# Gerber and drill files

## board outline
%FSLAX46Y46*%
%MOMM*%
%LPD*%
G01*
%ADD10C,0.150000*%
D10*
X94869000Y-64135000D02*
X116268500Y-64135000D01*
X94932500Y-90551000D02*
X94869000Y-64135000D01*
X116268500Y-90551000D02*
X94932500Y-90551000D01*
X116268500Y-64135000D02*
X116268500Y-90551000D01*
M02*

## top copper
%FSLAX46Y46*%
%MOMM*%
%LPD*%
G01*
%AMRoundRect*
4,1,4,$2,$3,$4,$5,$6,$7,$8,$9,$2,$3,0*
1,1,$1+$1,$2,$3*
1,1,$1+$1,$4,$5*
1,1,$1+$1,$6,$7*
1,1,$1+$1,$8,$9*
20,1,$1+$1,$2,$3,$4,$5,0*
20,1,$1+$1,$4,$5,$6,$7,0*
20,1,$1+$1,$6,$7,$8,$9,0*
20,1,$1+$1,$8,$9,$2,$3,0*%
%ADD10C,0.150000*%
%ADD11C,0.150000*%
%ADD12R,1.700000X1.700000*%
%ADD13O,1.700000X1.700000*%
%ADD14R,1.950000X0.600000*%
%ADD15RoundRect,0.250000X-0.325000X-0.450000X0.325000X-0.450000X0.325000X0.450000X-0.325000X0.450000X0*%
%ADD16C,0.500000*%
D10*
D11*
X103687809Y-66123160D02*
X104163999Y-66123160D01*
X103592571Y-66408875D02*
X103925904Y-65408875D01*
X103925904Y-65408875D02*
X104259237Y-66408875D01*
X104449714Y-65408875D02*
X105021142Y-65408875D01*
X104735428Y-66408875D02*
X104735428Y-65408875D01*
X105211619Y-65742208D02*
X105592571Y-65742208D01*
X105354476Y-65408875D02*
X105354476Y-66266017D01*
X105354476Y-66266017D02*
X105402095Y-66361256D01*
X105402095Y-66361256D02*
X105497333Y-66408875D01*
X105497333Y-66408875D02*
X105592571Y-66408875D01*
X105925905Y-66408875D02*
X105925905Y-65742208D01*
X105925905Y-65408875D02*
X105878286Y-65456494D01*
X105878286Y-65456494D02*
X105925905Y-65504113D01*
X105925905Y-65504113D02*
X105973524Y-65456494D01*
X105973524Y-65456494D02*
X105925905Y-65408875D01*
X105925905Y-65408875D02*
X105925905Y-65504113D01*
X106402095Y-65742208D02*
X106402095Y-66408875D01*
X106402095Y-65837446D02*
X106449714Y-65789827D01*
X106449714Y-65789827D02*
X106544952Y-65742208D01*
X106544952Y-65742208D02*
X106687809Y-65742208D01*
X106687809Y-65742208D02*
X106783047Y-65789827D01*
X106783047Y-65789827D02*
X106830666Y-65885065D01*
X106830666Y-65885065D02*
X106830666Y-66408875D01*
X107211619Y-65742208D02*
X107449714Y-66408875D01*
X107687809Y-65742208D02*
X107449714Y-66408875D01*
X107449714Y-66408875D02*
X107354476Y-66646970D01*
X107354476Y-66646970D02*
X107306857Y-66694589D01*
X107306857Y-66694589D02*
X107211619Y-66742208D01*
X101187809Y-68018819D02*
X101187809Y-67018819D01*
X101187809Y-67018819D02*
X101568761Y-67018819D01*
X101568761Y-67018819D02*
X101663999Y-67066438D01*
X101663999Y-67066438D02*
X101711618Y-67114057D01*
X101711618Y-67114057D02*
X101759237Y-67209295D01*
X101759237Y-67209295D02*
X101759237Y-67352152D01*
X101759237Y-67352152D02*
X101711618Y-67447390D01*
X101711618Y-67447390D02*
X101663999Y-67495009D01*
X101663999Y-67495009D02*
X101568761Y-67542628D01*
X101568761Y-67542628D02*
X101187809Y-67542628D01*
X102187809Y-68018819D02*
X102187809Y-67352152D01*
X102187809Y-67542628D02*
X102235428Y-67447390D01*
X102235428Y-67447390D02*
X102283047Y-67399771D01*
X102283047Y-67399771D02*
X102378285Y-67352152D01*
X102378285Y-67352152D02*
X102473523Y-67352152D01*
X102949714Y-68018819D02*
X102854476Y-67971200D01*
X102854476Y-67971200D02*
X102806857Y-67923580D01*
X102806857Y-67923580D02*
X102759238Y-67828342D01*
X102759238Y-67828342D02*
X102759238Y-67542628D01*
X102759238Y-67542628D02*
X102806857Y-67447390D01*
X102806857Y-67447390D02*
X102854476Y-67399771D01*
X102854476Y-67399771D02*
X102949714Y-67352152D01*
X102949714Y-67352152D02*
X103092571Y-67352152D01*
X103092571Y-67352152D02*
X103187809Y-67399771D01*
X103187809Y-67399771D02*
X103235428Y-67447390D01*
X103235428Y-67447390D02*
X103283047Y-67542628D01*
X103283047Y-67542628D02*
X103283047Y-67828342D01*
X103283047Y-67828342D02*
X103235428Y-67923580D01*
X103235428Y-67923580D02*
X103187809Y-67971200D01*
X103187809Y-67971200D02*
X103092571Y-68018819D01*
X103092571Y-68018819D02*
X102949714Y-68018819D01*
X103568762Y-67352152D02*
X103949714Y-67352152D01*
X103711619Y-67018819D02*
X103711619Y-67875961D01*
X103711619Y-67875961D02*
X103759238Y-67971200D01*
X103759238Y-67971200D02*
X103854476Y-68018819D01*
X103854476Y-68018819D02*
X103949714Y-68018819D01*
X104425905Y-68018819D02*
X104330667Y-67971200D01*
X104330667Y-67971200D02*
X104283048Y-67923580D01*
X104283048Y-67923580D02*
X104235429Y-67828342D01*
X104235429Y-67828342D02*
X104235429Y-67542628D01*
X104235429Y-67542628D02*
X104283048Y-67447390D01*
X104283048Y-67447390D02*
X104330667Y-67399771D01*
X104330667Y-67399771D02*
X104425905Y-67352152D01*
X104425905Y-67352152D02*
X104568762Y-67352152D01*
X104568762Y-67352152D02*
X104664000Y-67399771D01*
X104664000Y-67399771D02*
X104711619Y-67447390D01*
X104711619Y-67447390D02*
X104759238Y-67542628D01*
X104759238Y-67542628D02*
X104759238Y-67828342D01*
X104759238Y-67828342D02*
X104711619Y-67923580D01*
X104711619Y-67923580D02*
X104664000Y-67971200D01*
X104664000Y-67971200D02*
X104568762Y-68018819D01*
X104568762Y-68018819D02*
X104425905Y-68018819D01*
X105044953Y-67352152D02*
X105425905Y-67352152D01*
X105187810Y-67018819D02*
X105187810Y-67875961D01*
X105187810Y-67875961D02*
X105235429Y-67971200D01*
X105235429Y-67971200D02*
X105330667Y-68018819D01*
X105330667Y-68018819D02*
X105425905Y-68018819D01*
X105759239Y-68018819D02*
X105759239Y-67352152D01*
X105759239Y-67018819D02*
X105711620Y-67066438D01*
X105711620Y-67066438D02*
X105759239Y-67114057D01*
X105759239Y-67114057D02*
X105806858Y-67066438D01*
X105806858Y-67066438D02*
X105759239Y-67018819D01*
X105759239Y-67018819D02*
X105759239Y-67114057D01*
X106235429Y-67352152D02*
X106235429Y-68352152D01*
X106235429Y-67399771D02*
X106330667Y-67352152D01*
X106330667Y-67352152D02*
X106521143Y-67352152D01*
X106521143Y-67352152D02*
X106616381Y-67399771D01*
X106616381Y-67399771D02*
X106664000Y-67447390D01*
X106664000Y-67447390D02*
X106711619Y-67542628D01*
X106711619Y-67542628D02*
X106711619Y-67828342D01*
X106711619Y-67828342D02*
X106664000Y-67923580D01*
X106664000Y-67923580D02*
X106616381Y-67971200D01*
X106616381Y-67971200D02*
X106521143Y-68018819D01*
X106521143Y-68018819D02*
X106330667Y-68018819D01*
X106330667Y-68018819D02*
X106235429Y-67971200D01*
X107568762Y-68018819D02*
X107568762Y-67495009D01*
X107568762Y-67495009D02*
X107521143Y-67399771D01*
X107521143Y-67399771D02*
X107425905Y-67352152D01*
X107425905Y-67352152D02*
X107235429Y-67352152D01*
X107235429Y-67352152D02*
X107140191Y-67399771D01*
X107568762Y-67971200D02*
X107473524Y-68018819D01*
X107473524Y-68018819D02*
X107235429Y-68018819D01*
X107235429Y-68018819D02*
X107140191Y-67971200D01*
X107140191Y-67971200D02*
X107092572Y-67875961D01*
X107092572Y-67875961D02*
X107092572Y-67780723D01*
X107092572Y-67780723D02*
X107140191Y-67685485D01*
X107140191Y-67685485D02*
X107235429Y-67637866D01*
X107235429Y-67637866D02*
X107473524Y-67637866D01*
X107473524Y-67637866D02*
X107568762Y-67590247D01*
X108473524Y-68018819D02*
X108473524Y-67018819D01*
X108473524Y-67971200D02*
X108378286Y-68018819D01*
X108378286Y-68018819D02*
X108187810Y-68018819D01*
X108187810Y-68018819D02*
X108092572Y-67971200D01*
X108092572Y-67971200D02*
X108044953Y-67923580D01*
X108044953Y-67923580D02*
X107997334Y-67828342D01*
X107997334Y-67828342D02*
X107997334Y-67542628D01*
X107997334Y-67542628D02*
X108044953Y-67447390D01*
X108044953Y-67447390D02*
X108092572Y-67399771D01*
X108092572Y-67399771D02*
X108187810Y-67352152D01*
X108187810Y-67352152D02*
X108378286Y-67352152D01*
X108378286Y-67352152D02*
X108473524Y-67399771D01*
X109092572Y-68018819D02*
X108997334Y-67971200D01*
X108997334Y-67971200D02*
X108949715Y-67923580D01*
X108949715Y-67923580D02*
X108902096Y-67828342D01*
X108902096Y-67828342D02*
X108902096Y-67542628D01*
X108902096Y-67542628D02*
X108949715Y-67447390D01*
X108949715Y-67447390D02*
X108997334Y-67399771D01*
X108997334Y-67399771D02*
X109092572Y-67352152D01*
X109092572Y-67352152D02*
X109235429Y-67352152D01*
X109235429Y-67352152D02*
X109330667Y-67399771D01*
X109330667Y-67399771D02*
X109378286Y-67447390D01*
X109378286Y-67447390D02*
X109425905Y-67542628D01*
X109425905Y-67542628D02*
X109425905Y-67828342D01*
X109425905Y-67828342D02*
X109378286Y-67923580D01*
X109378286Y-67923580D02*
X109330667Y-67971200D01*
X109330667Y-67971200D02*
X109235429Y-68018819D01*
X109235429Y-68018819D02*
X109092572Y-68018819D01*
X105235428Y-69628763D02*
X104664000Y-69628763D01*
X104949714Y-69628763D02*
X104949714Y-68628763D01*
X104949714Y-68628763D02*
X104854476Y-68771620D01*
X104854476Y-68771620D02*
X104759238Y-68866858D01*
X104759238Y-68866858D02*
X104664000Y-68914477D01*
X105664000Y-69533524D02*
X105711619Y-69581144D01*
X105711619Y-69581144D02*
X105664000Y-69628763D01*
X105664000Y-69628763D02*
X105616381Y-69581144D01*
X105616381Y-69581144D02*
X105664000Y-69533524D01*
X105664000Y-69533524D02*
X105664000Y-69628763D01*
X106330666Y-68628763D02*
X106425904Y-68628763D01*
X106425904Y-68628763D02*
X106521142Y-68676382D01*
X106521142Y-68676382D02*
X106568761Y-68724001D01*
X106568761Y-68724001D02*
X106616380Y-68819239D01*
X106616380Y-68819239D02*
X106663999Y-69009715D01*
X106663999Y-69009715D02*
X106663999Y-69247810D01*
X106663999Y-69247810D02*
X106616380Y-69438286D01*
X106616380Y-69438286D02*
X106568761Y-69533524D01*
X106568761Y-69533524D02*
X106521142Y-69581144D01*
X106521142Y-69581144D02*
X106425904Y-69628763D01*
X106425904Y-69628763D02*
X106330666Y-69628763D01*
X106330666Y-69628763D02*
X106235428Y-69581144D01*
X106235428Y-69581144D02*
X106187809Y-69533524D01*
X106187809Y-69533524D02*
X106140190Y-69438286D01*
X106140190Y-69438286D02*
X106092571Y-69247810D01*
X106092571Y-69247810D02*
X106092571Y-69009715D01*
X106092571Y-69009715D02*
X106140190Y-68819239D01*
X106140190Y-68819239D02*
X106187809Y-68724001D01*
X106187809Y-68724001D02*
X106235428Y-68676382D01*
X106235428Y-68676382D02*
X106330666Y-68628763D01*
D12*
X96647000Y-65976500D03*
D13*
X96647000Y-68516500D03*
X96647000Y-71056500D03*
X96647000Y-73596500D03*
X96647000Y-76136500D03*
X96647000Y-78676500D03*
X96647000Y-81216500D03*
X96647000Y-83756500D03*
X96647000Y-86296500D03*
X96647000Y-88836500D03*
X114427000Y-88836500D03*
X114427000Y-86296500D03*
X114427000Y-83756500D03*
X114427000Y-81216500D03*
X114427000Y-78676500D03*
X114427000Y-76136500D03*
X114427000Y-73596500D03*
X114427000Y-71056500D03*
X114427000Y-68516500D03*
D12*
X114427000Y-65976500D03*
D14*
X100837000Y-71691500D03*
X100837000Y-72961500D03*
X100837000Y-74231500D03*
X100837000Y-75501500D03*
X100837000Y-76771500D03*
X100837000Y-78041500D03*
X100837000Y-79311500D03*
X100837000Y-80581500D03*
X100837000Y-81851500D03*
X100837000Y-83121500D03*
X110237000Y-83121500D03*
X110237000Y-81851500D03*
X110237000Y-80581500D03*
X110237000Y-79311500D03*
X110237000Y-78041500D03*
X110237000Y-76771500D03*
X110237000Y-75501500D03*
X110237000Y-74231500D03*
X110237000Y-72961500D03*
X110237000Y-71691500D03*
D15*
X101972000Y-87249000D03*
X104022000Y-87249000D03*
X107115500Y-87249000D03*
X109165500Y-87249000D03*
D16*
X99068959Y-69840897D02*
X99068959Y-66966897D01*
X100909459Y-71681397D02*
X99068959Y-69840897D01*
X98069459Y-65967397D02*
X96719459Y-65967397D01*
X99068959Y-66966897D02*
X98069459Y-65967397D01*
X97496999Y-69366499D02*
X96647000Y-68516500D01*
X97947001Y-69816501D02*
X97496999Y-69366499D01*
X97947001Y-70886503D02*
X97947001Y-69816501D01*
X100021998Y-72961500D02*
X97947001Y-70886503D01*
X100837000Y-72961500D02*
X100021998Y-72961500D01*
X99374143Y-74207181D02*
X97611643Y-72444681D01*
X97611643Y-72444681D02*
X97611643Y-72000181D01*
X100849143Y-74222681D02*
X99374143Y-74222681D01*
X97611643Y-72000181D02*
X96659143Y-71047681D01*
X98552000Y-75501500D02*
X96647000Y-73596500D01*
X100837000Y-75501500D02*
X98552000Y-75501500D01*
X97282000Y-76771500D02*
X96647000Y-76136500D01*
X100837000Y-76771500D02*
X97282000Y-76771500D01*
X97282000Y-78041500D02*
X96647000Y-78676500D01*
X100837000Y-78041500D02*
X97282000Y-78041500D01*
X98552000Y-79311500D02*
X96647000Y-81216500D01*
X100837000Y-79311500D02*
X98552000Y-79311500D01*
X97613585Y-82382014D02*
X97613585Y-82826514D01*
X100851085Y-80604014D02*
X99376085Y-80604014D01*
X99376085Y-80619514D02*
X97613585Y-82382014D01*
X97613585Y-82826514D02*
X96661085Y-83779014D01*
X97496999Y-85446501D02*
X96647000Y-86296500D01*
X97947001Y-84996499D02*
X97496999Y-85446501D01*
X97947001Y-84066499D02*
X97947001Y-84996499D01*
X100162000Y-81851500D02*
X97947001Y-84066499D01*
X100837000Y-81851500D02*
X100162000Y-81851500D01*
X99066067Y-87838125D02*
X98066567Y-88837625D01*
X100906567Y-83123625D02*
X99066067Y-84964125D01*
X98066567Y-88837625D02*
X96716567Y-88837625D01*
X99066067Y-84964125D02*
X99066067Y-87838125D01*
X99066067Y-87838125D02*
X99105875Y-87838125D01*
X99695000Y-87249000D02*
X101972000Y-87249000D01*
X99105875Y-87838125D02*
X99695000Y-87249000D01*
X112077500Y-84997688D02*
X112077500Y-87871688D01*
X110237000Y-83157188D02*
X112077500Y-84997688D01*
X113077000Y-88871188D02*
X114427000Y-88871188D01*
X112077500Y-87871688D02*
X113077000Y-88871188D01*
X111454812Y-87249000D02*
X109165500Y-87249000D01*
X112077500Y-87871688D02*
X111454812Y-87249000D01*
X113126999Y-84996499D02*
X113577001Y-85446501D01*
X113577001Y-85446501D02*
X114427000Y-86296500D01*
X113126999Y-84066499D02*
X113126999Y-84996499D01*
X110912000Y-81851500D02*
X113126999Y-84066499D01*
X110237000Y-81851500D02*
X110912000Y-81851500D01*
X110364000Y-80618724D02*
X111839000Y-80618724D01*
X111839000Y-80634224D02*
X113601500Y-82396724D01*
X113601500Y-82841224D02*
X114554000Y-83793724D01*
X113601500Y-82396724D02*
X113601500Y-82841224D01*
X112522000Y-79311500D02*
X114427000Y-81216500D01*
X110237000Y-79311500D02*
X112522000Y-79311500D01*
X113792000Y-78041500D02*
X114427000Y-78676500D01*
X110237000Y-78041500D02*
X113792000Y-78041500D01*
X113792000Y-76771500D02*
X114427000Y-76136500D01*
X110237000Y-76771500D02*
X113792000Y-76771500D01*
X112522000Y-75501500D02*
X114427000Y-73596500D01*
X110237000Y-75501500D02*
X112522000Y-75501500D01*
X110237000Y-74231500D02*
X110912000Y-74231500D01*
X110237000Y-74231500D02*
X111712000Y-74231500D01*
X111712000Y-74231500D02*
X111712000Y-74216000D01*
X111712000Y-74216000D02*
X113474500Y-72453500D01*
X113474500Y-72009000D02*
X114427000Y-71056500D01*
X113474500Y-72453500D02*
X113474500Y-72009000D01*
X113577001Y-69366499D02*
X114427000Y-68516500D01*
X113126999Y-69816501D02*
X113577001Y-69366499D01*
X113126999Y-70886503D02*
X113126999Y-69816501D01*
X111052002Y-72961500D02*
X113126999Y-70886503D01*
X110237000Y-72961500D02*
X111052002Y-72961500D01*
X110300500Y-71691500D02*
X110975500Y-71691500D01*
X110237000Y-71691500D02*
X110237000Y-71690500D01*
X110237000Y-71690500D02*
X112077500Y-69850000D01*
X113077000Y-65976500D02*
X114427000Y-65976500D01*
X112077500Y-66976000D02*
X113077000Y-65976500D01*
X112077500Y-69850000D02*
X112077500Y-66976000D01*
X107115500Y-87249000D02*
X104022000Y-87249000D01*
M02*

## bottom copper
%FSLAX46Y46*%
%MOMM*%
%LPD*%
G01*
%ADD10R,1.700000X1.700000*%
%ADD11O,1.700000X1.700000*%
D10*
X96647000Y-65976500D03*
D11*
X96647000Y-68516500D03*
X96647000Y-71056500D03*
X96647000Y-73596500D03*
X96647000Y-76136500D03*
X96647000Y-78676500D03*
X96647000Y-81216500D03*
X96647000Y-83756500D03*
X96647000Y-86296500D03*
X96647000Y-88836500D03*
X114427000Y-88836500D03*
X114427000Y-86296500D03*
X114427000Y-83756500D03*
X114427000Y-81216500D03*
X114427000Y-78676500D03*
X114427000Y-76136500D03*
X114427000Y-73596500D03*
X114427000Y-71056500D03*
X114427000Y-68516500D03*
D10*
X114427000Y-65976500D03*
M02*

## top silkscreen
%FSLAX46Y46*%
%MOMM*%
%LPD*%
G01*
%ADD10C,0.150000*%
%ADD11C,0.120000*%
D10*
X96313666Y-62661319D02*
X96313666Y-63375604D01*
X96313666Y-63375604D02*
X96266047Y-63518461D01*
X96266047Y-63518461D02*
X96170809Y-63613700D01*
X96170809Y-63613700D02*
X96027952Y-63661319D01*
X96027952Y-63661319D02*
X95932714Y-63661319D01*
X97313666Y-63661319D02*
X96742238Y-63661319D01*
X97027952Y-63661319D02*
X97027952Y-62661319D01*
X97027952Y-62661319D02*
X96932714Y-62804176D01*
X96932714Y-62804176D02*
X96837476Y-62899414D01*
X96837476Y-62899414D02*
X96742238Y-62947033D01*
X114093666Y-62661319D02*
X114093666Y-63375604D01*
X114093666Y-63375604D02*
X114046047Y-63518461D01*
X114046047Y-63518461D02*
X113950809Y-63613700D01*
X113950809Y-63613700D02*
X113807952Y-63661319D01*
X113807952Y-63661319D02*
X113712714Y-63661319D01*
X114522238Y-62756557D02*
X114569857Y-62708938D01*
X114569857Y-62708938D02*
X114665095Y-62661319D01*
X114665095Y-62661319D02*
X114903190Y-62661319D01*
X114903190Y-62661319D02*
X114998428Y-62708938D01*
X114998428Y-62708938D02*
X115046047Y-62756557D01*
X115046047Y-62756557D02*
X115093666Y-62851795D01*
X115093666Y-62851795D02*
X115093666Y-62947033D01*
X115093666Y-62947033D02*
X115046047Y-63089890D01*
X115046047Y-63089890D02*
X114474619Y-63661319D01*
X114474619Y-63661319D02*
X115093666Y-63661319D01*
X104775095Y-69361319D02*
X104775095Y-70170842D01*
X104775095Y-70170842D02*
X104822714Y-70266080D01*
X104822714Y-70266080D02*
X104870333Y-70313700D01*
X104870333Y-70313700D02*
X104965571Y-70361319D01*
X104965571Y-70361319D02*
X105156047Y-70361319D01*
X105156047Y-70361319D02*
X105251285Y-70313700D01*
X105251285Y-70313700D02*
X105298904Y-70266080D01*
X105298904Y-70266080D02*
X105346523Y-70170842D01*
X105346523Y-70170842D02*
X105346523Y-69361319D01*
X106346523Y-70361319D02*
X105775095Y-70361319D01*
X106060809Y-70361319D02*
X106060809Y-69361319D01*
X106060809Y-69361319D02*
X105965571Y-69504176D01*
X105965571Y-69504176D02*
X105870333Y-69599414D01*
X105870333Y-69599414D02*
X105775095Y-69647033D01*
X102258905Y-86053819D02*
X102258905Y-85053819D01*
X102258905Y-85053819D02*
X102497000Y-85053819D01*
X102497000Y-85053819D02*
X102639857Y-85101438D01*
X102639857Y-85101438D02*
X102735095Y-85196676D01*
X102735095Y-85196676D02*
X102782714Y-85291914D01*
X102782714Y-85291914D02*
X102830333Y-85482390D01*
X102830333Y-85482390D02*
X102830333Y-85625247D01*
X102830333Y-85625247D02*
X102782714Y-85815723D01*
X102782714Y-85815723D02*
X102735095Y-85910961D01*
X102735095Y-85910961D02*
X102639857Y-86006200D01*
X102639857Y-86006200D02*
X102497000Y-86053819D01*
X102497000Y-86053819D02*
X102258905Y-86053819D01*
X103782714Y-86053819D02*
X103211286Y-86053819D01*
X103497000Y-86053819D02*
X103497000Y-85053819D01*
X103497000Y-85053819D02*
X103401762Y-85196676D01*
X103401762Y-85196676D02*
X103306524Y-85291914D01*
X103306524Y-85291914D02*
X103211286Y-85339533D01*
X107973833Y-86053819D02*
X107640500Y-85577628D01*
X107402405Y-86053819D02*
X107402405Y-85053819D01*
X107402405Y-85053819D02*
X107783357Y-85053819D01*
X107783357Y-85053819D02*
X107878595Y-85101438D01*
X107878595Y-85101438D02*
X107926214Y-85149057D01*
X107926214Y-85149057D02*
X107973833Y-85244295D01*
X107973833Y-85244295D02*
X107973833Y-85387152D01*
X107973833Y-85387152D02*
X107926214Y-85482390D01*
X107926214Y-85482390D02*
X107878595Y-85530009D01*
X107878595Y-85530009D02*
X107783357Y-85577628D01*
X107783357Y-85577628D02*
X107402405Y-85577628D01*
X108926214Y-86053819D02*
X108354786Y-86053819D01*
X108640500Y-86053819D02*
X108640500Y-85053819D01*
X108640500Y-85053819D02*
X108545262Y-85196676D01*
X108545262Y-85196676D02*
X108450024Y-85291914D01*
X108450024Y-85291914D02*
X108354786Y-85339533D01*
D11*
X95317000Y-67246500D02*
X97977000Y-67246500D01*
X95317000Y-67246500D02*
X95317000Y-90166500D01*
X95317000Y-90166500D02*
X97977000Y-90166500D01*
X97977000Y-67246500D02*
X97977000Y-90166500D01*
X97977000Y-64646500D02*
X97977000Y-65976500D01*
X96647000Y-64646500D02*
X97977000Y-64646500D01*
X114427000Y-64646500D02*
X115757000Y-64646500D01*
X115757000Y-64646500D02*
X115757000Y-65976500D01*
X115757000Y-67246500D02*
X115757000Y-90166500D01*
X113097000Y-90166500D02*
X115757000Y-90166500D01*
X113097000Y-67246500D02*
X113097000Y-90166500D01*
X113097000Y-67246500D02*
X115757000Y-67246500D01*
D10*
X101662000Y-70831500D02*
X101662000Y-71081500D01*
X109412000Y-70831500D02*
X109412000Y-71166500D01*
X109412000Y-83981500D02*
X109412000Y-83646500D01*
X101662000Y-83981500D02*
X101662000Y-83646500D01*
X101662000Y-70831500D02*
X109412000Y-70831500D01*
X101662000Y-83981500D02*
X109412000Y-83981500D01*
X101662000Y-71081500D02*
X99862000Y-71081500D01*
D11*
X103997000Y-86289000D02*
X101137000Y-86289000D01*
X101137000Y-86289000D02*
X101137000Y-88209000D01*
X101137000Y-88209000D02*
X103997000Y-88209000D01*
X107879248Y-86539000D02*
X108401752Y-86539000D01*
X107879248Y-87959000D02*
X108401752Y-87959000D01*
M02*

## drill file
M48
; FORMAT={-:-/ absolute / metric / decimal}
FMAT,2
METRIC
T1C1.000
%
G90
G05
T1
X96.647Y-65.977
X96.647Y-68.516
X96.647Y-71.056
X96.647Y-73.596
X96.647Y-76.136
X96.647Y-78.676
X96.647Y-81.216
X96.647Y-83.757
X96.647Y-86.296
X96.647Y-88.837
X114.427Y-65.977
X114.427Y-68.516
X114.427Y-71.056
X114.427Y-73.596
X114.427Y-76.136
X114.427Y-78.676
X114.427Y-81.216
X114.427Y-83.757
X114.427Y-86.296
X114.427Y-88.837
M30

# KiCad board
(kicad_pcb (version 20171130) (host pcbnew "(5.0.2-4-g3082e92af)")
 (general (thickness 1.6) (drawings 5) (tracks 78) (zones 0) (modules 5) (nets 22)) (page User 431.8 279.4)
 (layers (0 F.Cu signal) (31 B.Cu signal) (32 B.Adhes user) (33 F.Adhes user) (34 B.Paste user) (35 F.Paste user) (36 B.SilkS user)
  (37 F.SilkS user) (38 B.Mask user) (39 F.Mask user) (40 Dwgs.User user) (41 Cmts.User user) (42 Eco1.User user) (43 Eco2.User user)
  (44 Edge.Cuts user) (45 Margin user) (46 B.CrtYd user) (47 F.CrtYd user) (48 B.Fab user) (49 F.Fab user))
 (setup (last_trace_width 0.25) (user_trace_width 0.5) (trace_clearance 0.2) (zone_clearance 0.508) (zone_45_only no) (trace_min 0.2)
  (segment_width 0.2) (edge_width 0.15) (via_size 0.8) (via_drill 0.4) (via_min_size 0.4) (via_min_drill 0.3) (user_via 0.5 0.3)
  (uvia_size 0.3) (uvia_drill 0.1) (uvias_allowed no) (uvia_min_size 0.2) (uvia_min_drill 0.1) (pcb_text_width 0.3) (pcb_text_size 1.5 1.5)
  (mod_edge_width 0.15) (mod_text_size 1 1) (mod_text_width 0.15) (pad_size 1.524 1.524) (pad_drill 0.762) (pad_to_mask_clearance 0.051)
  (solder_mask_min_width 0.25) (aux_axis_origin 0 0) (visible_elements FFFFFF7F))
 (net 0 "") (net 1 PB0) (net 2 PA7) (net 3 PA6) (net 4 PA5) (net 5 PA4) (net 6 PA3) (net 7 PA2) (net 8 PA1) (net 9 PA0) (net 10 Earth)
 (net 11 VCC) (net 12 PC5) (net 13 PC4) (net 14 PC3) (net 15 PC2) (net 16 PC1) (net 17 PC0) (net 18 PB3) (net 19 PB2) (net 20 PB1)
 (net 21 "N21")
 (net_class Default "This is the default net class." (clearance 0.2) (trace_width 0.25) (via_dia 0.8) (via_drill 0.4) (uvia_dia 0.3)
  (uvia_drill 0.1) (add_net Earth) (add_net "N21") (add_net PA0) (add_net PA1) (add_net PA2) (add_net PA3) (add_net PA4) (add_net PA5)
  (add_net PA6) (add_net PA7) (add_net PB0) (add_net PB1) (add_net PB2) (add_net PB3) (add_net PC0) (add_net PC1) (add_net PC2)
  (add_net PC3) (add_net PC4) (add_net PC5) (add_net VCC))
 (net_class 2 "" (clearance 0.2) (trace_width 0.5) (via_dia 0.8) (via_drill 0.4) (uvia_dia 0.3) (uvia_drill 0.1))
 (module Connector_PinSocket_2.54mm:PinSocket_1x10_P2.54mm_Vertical (layer F.Cu) (at 96.647 65.9765)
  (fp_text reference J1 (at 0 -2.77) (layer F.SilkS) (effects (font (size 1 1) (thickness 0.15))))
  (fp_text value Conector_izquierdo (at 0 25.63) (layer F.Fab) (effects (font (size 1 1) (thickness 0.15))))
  (fp_line (start -1.33 1.27) (end 1.33 1.27) (layer F.SilkS) (width 0.12))
  (fp_line (start -1.33 1.27) (end -1.33 24.19) (layer F.SilkS) (width 0.12))
  (fp_line (start -1.33 24.19) (end 1.33 24.19) (layer F.SilkS) (width 0.12))
  (fp_line (start 1.33 1.27) (end 1.33 24.19) (layer F.SilkS) (width 0.12))
  (fp_line (start 1.33 -1.33) (end 1.33 0) (layer F.SilkS) (width 0.12))
  (fp_line (start 0 -1.33) (end 1.33 -1.33) (layer F.SilkS) (width 0.12))
  (pad 1 thru_hole rect (at 0 0) (size 1.7 1.7) (drill 1) (layers *.Cu *.Mask) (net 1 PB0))
  (pad 2 thru_hole oval (at 0 2.54) (size 1.7 1.7) (drill 1) (layers *.Cu *.Mask) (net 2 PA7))
  (pad 3 thru_hole oval (at 0 5.08) (size 1.7 1.7) (drill 1) (layers *.Cu *.Mask) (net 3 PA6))
  (pad 4 thru_hole oval (at 0 7.62) (size 1.7 1.7) (drill 1) (layers *.Cu *.Mask) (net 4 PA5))
  (pad 5 thru_hole oval (at 0 10.16) (size 1.7 1.7) (drill 1) (layers *.Cu *.Mask) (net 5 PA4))
  (pad 6 thru_hole oval (at 0 12.7) (size 1.7 1.7) (drill 1) (layers *.Cu *.Mask) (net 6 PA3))
  (pad 7 thru_hole oval (at 0 15.24) (size 1.7 1.7) (drill 1) (layers *.Cu *.Mask) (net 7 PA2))
  (pad 8 thru_hole oval (at 0 17.78) (size 1.7 1.7) (drill 1) (layers *.Cu *.Mask) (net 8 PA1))
  (pad 9 thru_hole oval (at 0 20.32) (size 1.7 1.7) (drill 1) (layers *.Cu *.Mask) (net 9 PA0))
  (pad 10 thru_hole oval (at 0 22.86) (size 1.7 1.7) (drill 1) (layers *.Cu *.Mask) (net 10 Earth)))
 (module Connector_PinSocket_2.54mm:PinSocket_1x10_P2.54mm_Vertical (layer F.Cu) (at 114.427 65.9765)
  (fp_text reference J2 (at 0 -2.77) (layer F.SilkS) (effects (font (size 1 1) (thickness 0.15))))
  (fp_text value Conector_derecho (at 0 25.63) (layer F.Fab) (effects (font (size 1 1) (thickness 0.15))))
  (fp_line (start 0 -1.33) (end 1.33 -1.33) (layer F.SilkS) (width 0.12))
  (fp_line (start 1.33 -1.33) (end 1.33 0) (layer F.SilkS) (width 0.12))
  (fp_line (start 1.33 1.27) (end 1.33 24.19) (layer F.SilkS) (width 0.12))
  (fp_line (start -1.33 24.19) (end 1.33 24.19) (layer F.SilkS) (width 0.12))
  (fp_line (start -1.33 1.27) (end -1.33 24.19) (layer F.SilkS) (width 0.12))
  (fp_line (start -1.33 1.27) (end 1.33 1.27) (layer F.SilkS) (width 0.12))
  (pad 10 thru_hole oval (at 0 22.86) (size 1.7 1.7) (drill 1) (layers *.Cu *.Mask) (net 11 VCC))
  (pad 9 thru_hole oval (at 0 20.32) (size 1.7 1.7) (drill 1) (layers *.Cu *.Mask) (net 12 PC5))
  (pad 8 thru_hole oval (at 0 17.78) (size 1.7 1.7) (drill 1) (layers *.Cu *.Mask) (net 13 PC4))
  (pad 7 thru_hole oval (at 0 15.24) (size 1.7 1.7) (drill 1) (layers *.Cu *.Mask) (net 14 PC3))
  (pad 6 thru_hole oval (at 0 12.7) (size 1.7 1.7) (drill 1) (layers *.Cu *.Mask) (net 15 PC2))
  (pad 5 thru_hole oval (at 0 10.16) (size 1.7 1.7) (drill 1) (layers *.Cu *.Mask) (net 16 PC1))
  (pad 4 thru_hole oval (at 0 7.62) (size 1.7 1.7) (drill 1) (layers *.Cu *.Mask) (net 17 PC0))
  (pad 3 thru_hole oval (at 0 5.08) (size 1.7 1.7) (drill 1) (layers *.Cu *.Mask) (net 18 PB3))
  (pad 2 thru_hole oval (at 0 2.54) (size 1.7 1.7) (drill 1) (layers *.Cu *.Mask) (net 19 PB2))
  (pad 1 thru_hole rect (at 0 0) (size 1.7 1.7) (drill 1) (layers *.Cu *.Mask) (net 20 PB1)))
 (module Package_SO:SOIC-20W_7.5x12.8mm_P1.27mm (layer F.Cu) (at 105.537 77.4065)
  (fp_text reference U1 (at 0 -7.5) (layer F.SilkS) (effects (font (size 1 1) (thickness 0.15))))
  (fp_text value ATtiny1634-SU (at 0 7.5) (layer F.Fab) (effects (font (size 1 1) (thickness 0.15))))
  (fp_line (start -3.875 -6.575) (end -3.875 -6.325) (layer F.SilkS) (width 0.15))
  (fp_line (start 3.875 -6.575) (end 3.875 -6.24) (layer F.SilkS) (width 0.15))
  (fp_line (start 3.875 6.575) (end 3.875 6.24) (layer F.SilkS) (width 0.15))
  (fp_line (start -3.875 6.575) (end -3.875 6.24) (layer F.SilkS) (width 0.15))
  (fp_line (start -3.875 -6.575) (end 3.875 -6.575) (layer F.SilkS) (width 0.15))
  (fp_line (start -3.875 6.575) (end 3.875 6.575) (layer F.SilkS) (width 0.15))
  (fp_line (start -3.875 -6.325) (end -5.675 -6.325) (layer F.SilkS) (width 0.15))
  (pad 1 smd rect (at -4.7 -5.715) (size 1.95 0.6) (layers F.Cu F.Paste F.Mask) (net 1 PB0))
  (pad 2 smd rect (at -4.7 -4.445) (size 1.95 0.6) (layers F.Cu F.Paste F.Mask) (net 2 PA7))
  (pad 3 smd rect (at -4.7 -3.175) (size 1.95 0.6) (layers F.Cu F.Paste F.Mask) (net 3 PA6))
  (pad 4 smd rect (at -4.7 -1.905) (size 1.95 0.6) (layers F.Cu F.Paste F.Mask) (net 4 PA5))
  (pad 5 smd rect (at -4.7 -0.635) (size 1.95 0.6) (layers F.Cu F.Paste F.Mask) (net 5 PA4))
  (pad 6 smd rect (at -4.7 0.635) (size 1.95 0.6) (layers F.Cu F.Paste F.Mask) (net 6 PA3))
  (pad 7 smd rect (at -4.7 1.905) (size 1.95 0.6) (layers F.Cu F.Paste F.Mask) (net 7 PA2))
  (pad 8 smd rect (at -4.7 3.175) (size 1.95 0.6) (layers F.Cu F.Paste F.Mask) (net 8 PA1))
  (pad 9 smd rect (at -4.7 4.445) (size 1.95 0.6) (layers F.Cu F.Paste F.Mask) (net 9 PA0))
  (pad 10 smd rect (at -4.7 5.715) (size 1.95 0.6) (layers F.Cu F.Paste F.Mask) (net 10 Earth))
  (pad 11 smd rect (at 4.7 5.715) (size 1.95 0.6) (layers F.Cu F.Paste F.Mask) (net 11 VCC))
  (pad 12 smd rect (at 4.7 4.445) (size 1.95 0.6) (layers F.Cu F.Paste F.Mask) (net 12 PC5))
  (pad 13 smd rect (at 4.7 3.175) (size 1.95 0.6) (layers F.Cu F.Paste F.Mask) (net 13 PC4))
  (pad 14 smd rect (at 4.7 1.905) (size 1.95 0.6) (layers F.Cu F.Paste F.Mask) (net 14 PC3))
  (pad 15 smd rect (at 4.7 0.635) (size 1.95 0.6) (layers F.Cu F.Paste F.Mask) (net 15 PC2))
  (pad 16 smd rect (at 4.7 -0.635) (size 1.95 0.6) (layers F.Cu F.Paste F.Mask) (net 16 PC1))
  (pad 17 smd rect (at 4.7 -1.905) (size 1.95 0.6) (layers F.Cu F.Paste F.Mask) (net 17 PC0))
  (pad 18 smd rect (at 4.7 -3.175) (size 1.95 0.6) (layers F.Cu F.Paste F.Mask) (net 18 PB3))
  (pad 19 smd rect (at 4.7 -4.445) (size 1.95 0.6) (layers F.Cu F.Paste F.Mask) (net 19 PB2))
  (pad 20 smd rect (at 4.7 -5.715) (size 1.95 0.6) (layers F.Cu F.Paste F.Mask) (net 20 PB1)))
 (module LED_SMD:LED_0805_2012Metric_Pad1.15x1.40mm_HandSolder (layer F.Cu) (at 102.997 87.249)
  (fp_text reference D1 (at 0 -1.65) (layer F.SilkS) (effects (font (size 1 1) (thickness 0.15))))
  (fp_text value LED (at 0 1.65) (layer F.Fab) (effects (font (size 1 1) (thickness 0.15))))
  (fp_line (start 1 -0.96) (end -1.86 -0.96) (layer F.SilkS) (width 0.12))
  (fp_line (start -1.86 -0.96) (end -1.86 0.96) (layer F.SilkS) (width 0.12))
  (fp_line (start -1.86 0.96) (end 1 0.96) (layer F.SilkS) (width 0.12))
  (pad 1 smd roundrect (at -1.025 0) (size 1.15 1.4) (layers F.Cu F.Paste F.Mask) (roundrect_rratio 0.217391) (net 10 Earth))
  (pad 2 smd roundrect (at 1.025 0) (size 1.15 1.4) (layers F.Cu F.Paste F.Mask) (roundrect_rratio 0.217391) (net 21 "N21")))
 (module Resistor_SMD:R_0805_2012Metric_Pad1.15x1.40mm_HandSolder (layer F.Cu) (at 108.1405 87.249)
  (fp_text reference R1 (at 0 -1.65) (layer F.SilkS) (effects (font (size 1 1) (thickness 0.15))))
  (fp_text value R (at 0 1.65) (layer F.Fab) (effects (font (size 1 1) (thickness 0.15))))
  (fp_line (start -0.261252 -0.71) (end 0.261252 -0.71) (layer F.SilkS) (width 0.12))
  (fp_line (start -0.261252 0.71) (end 0.261252 0.71) (layer F.SilkS) (width 0.12))
  (pad 1 smd roundrect (at -1.025 0) (size 1.15 1.4) (layers F.Cu F.Paste F.Mask) (roundrect_rratio 0.217391) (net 21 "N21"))
  (pad 2 smd roundrect (at 1.025 0) (size 1.15 1.4) (layers F.Cu F.Paste F.Mask) (roundrect_rratio 0.217391) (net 11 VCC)))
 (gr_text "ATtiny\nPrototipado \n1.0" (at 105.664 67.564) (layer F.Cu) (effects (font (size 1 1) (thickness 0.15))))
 (gr_line (start 94.869 64.135) (end 116.2685 64.135) (layer Edge.Cuts) (width 0.15))
 (gr_line (start 94.9325 90.551) (end 94.869 64.135) (layer Edge.Cuts) (width 0.15))
 (gr_line (start 116.2685 90.551) (end 94.9325 90.551) (layer Edge.Cuts) (width 0.15))
 (gr_line (start 116.2685 64.135) (end 116.2685 90.551) (layer Edge.Cuts) (width 0.15))
 (segment (start 99.068959 69.840897) (end 99.068959 66.966897) (width 0.5) (layer F.Cu) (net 1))
 (segment (start 100.909459 71.681397) (end 99.068959 69.840897) (width 0.5) (layer F.Cu) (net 1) (status 10))
 (segment (start 98.069459 65.967397) (end 96.719459 65.967397) (width 0.5) (layer F.Cu) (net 1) (status 20))
 (segment (start 99.068959 66.966897) (end 98.069459 65.967397) (width 0.5) (layer F.Cu) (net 1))
 (segment (start 97.496999 69.366499) (end 96.647 68.5165) (width 0.5) (layer F.Cu) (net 2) (status 30))
 (segment (start 97.947001 69.816501) (end 97.496999 69.366499) (width 0.5) (layer F.Cu) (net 2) (status 20))
 (segment (start 97.947001 70.886503) (end 97.947001 69.816501) (width 0.5) (layer F.Cu) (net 2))
 (segment (start 100.021998 72.9615) (end 97.947001 70.886503) (width 0.5) (layer F.Cu) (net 2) (status 10))
 (segment (start 100.837 72.9615) (end 100.021998 72.9615) (width 0.5) (layer F.Cu) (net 2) (status 30))
 (segment (start 99.374143 74.207181) (end 97.611643 72.444681) (width 0.5) (layer F.Cu) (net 3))
 (segment (start 97.611643 72.444681) (end 97.611643 72.000181) (width 0.5) (layer F.Cu) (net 3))
 (segment (start 100.849143 74.222681) (end 99.374143 74.222681) (width 0.5) (layer F.Cu) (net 3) (status 10))
 (segment (start 97.611643 72.000181) (end 96.659143 71.047681) (width 0.5) (layer F.Cu) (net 3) (status 20))
 (segment (start 98.552 75.5015) (end 96.647 73.5965) (width 0.5) (layer F.Cu) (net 4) (status 20))
 (segment (start 100.837 75.5015) (end 98.552 75.5015) (width 0.5) (layer F.Cu) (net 4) (status 10))
 (segment (start 97.282 76.7715) (end 96.647 76.1365) (width 0.5) (layer F.Cu) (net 5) (status 30))
 (segment (start 100.837 76.7715) (end 97.282 76.7715) (width 0.5) (layer F.Cu) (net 5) (status 30))
 (segment (start 97.282 78.0415) (end 96.647 78.6765) (width 0.5) (layer F.Cu) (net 6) (status 30))
 (segment (start 100.837 78.0415) (end 97.282 78.0415) (width 0.5) (layer F.Cu) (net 6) (status 30))
 (segment (start 98.552 79.3115) (end 96.647 81.2165) (width 0.5) (layer F.Cu) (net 7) (status 20))
 (segment (start 100.837 79.3115) (end 98.552 79.3115) (width 0.5) (layer F.Cu) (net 7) (status 10))
 (segment (start 97.613585 82.382014) (end 97.613585 82.826514) (width 0.5) (layer F.Cu) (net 8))
 (segment (start 100.851085 80.604014) (end 99.376085 80.604014) (width 0.5) (layer F.Cu) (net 8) (status 10))
 (segment (start 99.376085 80.619514) (end 97.613585 82.382014) (width 0.5) (layer F.Cu) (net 8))
 (segment (start 97.613585 82.826514) (end 96.661085 83.779014) (width 0.5) (layer F.Cu) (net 8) (status 20))
 (segment (start 97.496999 85.446501) (end 96.647 86.2965) (width 0.5) (layer F.Cu) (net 9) (status 30))
 (segment (start 97.947001 84.996499) (end 97.496999 85.446501) (width 0.5) (layer F.Cu) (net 9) (status 20))
 (segment (start 97.947001 84.066499) (end 97.947001 84.996499) (width 0.5) (layer F.Cu) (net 9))
 (segment (start 100.162 81.8515) (end 97.947001 84.066499) (width 0.5) (layer F.Cu) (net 9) (status 10))
 (segment (start 100.837 81.8515) (end 100.162 81.8515) (width 0.5) (layer F.Cu) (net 9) (status 30))
 (segment (start 99.066067 87.838125) (end 98.066567 88.837625) (width 0.5) (layer F.Cu) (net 10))
 (segment (start 100.906567 83.123625) (end 99.066067 84.964125) (width 0.5) (layer F.Cu) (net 10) (status 10))
 (segment (start 98.066567 88.837625) (end 96.716567 88.837625) (width 0.5) (layer F.Cu) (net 10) (status 20))
 (segment (start 99.066067 84.964125) (end 99.066067 87.838125) (width 0.5) (layer F.Cu) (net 10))
 (segment (start 99.066067 87.838125) (end 99.105875 87.838125) (width 0.5) (layer F.Cu) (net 10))
 (segment (start 99.695 87.249) (end 101.972 87.249) (width 0.5) (layer F.Cu) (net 10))
 (segment (start 99.105875 87.838125) (end 99.695 87.249) (width 0.5) (layer F.Cu) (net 10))
 (segment (start 112.0775 84.997688) (end 112.0775 87.871688) (width 0.5) (layer F.Cu) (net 11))
 (segment (start 110.237 83.157188) (end 112.0775 84.997688) (width 0.5) (layer F.Cu) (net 11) (status 10))
 (segment (start 113.077 88.871188) (end 114.427 88.871188) (width 0.5) (layer F.Cu) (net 11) (status 20))
 (segment (start 112.0775 87.871688) (end 113.077 88.871188) (width 0.5) (layer F.Cu) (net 11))
 (segment (start 111.454812 87.249) (end 109.1655 87.249) (width 0.5) (layer F.Cu) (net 11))
 (segment (start 112.0775 87.871688) (end 111.454812 87.249) (width 0.5) (layer F.Cu) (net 11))
 (segment (start 113.126999 84.996499) (end 113.577001 85.446501) (width 0.5) (layer F.Cu) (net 12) (status 20))
 (segment (start 113.577001 85.446501) (end 114.427 86.2965) (width 0.5) (layer F.Cu) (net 12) (status 30))
 (segment (start 113.126999 84.066499) (end 113.126999 84.996499) (width 0.5) (layer F.Cu) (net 12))
 (segment (start 110.912 81.8515) (end 113.126999 84.066499) (width 0.5) (layer F.Cu) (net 12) (status 10))
 (segment (start 110.237 81.8515) (end 110.912 81.8515) (width 0.5) (layer F.Cu) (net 12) (status 30))
 (segment (start 110.364 80.618724) (end 111.839 80.618724) (width 0.5) (layer F.Cu) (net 13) (status 10))
 (segment (start 111.839 80.634224) (end 113.6015 82.396724) (width 0.5) (layer F.Cu) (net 13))
 (segment (start 113.6015 82.841224) (end 114.554 83.793724) (width 0.5) (layer F.Cu) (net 13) (status 20))
 (segment (start 113.6015 82.396724) (end 113.6015 82.841224) (width 0.5) (layer F.Cu) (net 13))
 (segment (start 112.522 79.3115) (end 114.427 81.2165) (width 0.5) (layer F.Cu) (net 14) (status 20))
 (segment (start 110.237 79.3115) (end 112.522 79.3115) (width 0.5) (layer F.Cu) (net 14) (status 10))
 (segment (start 113.792 78.0415) (end 114.427 78.6765) (width 0.5) (layer F.Cu) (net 15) (status 30))
 (segment (start 110.237 78.0415) (end 113.792 78.0415) (width 0.5) (layer F.Cu) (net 15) (status 30))
 (segment (start 113.792 76.7715) (end 114.427 76.1365) (width 0.5) (layer F.Cu) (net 16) (status 30))
 (segment (start 110.237 76.7715) (end 113.792 76.7715) (width 0.5) (layer F.Cu) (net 16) (status 30))
 (segment (start 112.522 75.5015) (end 114.427 73.5965) (width 0.5) (layer F.Cu) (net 17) (status 20))
 (segment (start 110.237 75.5015) (end 112.522 75.5015) (width 0.5) (layer F.Cu) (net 17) (status 10))
 (segment (start 110.237 74.2315) (end 110.912 74.2315) (width 0.5) (layer F.Cu) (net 18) (status 30))
 (segment (start 110.237 74.2315) (end 111.712 74.2315) (width 0.5) (layer F.Cu) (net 18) (status 10))
 (segment (start 111.712 74.2315) (end 111.712 74.216) (width 0.5) (layer F.Cu) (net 18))
 (segment (start 111.712 74.216) (end 113.4745 72.4535) (width 0.5) (layer F.Cu) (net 18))
 (segment (start 113.4745 72.009) (end 114.427 71.0565) (width 0.5) (layer F.Cu) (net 18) (status 20))
 (segment (start 113.4745 72.4535) (end 113.4745 72.009) (width 0.5) (layer F.Cu) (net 18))
 (segment (start 113.577001 69.366499) (end 114.427 68.5165) (width 0.5) (layer F.Cu) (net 19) (status 30))
 (segment (start 113.126999 69.816501) (end 113.577001 69.366499) (width 0.5) (layer F.Cu) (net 19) (status 20))
 (segment (start 113.126999 70.886503) (end 113.126999 69.816501) (width 0.5) (layer F.Cu) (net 19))
 (segment (start 111.052002 72.9615) (end 113.126999 70.886503) (width 0.5) (layer F.Cu) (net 19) (status 10))
 (segment (start 110.237 72.9615) (end 111.052002 72.9615) (width 0.5) (layer F.Cu) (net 19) (status 30))
 (segment (start 110.3005 71.6915) (end 110.9755 71.6915) (width 0.5) (layer F.Cu) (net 20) (status 30))
 (segment (start 110.237 71.6915) (end 110.237 71.6905) (width 0.5) (layer F.Cu) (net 20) (status 30))
 (segment (start 110.237 71.6905) (end 112.0775 69.85) (width 0.5) (layer F.Cu) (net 20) (status 10))
 (segment (start 113.077 65.9765) (end 114.427 65.9765) (width 0.5) (layer F.Cu) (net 20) (status 20))
 (segment (start 112.0775 66.976) (end 113.077 65.9765) (width 0.5) (layer F.Cu) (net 20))
 (segment (start 112.0775 69.85) (end 112.0775 66.976) (width 0.5) (layer F.Cu) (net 20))
 (segment (start 107.1155 87.249) (end 104.022 87.249) (width 0.5) (layer F.Cu) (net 21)))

